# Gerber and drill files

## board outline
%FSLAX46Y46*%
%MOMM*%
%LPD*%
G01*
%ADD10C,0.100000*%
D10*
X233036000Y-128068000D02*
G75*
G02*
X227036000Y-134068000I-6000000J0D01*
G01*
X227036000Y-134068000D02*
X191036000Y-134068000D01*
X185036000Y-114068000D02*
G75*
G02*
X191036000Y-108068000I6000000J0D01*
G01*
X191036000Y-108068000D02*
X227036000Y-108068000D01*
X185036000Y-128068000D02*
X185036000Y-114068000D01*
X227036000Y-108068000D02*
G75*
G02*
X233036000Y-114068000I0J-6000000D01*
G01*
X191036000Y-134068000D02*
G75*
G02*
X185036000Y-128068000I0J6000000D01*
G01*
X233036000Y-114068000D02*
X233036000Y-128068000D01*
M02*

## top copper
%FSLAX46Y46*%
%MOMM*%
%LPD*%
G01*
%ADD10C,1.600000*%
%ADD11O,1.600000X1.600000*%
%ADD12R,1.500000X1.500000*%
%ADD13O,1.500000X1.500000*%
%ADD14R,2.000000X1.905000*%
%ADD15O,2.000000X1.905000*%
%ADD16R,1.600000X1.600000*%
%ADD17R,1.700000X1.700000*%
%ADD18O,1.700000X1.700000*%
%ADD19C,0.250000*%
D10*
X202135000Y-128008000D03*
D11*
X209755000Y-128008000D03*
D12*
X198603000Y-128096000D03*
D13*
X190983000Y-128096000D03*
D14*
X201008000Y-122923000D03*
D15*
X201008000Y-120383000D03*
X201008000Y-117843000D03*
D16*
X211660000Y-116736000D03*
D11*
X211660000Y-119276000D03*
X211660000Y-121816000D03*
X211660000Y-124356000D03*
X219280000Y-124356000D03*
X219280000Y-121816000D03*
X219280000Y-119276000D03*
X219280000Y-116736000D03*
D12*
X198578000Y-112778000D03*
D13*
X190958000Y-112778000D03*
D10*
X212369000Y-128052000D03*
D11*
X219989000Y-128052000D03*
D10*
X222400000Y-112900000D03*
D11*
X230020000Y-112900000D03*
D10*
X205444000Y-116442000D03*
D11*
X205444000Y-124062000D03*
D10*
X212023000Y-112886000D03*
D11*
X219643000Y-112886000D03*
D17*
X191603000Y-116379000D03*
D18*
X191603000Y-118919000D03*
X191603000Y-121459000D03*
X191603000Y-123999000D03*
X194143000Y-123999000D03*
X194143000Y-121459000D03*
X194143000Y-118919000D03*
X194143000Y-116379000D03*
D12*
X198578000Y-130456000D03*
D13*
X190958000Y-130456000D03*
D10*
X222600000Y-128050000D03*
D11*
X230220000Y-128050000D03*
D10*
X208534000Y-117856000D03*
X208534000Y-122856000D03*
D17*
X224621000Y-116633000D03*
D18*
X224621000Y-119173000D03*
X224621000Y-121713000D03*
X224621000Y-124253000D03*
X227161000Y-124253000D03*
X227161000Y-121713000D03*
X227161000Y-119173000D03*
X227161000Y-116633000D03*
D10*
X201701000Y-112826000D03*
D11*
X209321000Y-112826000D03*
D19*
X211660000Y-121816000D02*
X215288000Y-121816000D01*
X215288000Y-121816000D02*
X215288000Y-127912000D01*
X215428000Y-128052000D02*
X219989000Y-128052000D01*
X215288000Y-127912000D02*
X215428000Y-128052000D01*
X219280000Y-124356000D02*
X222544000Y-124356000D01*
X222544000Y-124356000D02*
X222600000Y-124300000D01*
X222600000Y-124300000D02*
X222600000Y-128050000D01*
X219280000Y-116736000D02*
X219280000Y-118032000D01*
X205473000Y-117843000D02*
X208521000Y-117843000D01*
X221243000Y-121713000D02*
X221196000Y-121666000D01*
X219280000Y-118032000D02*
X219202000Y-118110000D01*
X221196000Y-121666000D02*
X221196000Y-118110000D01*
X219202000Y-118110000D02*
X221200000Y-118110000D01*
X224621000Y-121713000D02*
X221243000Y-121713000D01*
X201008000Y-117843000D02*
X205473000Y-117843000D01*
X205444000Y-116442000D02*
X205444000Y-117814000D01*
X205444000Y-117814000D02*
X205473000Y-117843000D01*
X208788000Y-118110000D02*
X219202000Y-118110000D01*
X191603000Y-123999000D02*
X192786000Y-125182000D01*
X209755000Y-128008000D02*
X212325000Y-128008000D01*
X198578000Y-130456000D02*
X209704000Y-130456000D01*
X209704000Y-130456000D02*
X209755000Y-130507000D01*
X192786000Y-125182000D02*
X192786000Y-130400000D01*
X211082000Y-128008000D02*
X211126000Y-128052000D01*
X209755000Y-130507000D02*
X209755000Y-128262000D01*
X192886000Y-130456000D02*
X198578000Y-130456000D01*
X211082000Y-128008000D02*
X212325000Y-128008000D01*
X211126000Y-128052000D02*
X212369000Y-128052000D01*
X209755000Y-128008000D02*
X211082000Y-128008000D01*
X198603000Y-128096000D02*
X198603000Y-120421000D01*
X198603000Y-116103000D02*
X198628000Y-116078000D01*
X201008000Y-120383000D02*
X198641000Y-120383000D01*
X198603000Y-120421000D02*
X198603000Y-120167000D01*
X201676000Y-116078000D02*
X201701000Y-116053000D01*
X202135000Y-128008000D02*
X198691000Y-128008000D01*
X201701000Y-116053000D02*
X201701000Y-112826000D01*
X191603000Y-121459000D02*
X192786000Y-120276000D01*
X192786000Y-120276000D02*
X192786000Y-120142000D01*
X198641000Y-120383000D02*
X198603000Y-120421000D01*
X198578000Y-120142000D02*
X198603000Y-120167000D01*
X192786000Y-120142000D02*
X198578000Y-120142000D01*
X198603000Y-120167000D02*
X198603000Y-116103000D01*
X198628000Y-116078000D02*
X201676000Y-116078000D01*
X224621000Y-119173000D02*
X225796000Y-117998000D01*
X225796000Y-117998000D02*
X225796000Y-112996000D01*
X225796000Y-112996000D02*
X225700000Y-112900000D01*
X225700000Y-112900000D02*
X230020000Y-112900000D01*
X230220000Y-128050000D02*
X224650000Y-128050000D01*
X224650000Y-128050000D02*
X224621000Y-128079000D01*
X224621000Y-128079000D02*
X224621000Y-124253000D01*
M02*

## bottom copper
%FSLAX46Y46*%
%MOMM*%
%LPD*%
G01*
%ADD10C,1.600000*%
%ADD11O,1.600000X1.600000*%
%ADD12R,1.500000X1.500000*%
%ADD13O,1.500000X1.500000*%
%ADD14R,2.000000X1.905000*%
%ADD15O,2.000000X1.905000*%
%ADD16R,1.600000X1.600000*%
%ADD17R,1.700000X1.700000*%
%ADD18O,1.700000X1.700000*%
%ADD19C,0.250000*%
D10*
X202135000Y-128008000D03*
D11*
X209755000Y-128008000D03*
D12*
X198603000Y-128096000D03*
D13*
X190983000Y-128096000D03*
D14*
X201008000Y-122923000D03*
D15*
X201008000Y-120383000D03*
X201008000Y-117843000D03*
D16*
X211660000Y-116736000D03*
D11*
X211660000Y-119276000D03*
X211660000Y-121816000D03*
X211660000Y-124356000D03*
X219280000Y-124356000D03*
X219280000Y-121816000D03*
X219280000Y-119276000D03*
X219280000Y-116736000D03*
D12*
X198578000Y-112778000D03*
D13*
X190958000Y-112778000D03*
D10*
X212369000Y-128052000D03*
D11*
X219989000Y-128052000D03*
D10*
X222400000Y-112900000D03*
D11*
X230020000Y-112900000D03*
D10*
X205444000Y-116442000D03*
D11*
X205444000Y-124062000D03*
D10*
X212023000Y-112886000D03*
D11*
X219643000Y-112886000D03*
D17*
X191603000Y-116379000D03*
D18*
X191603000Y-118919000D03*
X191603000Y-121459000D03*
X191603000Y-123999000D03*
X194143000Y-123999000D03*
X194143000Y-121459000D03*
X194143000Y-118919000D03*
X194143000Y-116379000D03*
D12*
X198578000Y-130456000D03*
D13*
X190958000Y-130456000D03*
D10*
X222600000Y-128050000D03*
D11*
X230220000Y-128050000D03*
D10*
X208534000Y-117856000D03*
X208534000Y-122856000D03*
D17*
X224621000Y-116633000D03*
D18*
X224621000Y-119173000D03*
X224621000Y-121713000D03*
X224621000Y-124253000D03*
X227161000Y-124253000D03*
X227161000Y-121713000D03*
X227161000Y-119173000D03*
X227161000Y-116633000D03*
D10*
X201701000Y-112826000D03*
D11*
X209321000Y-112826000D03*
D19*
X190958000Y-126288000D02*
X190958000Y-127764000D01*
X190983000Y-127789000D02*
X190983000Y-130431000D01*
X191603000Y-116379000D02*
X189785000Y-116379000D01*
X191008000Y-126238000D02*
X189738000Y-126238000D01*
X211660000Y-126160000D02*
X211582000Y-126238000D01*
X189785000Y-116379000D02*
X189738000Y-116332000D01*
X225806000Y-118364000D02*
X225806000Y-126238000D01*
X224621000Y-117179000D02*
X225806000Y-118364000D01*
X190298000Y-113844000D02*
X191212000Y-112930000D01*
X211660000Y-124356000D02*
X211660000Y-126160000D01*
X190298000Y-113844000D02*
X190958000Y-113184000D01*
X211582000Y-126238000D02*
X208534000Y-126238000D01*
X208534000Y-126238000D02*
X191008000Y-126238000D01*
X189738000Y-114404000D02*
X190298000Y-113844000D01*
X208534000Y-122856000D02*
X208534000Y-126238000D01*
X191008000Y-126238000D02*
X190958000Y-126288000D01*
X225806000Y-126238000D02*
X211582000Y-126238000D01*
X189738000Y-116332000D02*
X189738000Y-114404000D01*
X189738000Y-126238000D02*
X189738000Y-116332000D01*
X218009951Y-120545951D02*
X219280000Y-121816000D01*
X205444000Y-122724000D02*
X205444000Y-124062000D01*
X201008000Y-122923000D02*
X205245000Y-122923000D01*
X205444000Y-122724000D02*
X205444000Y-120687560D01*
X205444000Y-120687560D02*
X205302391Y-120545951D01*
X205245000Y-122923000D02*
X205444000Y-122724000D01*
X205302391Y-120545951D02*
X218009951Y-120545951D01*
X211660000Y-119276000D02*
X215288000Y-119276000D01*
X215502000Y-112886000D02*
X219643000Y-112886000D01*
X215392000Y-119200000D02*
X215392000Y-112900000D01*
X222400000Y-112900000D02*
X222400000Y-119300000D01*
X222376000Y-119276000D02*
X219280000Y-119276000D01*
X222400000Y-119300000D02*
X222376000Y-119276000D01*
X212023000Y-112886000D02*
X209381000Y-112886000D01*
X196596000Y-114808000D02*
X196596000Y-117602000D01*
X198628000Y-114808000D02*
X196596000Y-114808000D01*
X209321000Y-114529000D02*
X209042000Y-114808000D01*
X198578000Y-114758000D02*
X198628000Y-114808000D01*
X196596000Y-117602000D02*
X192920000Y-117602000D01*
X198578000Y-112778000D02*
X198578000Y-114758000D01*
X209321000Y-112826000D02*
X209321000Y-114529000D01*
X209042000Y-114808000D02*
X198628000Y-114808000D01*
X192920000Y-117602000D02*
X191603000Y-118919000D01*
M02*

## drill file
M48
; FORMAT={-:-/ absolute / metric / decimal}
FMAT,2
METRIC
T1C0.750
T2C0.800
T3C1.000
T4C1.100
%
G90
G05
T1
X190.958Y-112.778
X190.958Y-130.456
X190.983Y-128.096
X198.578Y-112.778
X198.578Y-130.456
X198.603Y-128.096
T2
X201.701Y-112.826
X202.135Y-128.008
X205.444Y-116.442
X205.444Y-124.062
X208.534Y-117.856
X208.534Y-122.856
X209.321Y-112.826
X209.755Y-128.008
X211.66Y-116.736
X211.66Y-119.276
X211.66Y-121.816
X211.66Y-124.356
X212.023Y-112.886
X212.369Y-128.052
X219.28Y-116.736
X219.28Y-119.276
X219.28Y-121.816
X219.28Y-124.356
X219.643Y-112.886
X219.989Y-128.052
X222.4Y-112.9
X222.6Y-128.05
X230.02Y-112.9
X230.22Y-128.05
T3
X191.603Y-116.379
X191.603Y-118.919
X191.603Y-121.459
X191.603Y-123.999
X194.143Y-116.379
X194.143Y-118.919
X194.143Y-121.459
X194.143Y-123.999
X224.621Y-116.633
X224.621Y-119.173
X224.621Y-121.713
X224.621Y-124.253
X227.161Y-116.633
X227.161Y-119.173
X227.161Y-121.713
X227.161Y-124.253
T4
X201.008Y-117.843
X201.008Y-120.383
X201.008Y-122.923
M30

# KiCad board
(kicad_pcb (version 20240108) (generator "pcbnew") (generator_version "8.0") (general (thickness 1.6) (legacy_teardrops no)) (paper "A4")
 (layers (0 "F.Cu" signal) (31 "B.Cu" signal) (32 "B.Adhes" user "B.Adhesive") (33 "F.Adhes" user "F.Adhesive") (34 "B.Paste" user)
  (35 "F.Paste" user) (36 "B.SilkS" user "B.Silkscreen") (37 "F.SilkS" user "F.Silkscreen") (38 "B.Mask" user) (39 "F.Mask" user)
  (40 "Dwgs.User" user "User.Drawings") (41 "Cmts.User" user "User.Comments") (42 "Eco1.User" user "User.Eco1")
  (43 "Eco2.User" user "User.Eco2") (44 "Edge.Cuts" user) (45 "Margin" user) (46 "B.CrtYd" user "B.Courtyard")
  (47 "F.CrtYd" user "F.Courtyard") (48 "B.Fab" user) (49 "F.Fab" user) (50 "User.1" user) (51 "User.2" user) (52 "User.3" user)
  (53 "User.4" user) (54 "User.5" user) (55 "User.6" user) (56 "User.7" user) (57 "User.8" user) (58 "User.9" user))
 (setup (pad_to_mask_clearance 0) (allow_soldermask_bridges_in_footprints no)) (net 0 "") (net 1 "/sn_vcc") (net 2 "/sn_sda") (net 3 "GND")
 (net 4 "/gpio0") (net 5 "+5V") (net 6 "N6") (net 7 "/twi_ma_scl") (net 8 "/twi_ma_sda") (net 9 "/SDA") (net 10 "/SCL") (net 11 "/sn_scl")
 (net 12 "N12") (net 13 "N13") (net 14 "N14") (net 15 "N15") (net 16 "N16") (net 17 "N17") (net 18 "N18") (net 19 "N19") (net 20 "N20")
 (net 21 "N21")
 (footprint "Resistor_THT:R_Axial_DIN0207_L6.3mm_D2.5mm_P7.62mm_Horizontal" (layer "F.Cu") (at 202.135 128.008)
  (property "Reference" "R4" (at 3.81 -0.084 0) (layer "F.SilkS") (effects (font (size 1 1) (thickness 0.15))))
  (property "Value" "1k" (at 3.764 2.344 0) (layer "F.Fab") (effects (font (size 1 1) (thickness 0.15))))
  (pad "1" thru_hole circle (at 0 0) (size 1.6 1.6) (drill 0.8) (layers "*.Cu" "*.Mask") (remove_unused_layers no) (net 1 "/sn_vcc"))
  (pad "2" thru_hole oval (at 7.62 0) (size 1.6 1.6) (drill 0.8) (layers "*.Cu" "*.Mask") (remove_unused_layers no) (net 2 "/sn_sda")))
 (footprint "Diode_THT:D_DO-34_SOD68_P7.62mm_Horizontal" (layer "F.Cu") (at 198.603 128.096 180)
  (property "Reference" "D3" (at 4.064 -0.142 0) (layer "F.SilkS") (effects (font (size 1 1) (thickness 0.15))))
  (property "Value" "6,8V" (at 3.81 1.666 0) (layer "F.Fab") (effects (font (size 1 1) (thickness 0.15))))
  (pad "1" thru_hole rect (at 0 0 180) (size 1.5 1.5) (drill 0.75) (layers "*.Cu" "*.Mask") (remove_unused_layers no) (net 1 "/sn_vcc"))
  (pad "2" thru_hole oval (at 7.62 0 180) (size 1.5 1.5) (drill 0.75) (layers "*.Cu" "*.Mask") (remove_unused_layers no) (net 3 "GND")))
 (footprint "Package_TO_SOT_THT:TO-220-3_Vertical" (layer "F.Cu") (at 201.008 122.923 90)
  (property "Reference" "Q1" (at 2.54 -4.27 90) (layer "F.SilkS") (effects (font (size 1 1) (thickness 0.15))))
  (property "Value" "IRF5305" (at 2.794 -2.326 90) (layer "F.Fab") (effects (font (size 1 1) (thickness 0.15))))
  (pad "1" thru_hole rect (at 0 0 90) (size 1.905 2) (drill 1.1) (layers "*.Cu" "*.Mask") (remove_unused_layers no) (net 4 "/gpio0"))
  (pad "2" thru_hole oval (at 2.54 0 90) (size 1.905 2) (drill 1.1) (layers "*.Cu" "*.Mask") (remove_unused_layers no) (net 1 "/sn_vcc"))
  (pad "3" thru_hole oval (at 5.08 0 90) (size 1.905 2) (drill 1.1) (layers "*.Cu" "*.Mask") (remove_unused_layers no) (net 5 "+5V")))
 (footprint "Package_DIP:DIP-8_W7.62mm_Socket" (layer "F.Cu") (at 211.66 116.736)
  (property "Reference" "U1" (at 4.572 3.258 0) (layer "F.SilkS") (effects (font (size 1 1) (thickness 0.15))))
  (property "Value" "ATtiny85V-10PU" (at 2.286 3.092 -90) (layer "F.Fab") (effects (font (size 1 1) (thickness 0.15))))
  (pad "1" thru_hole rect (at 0 0) (size 1.6 1.6) (drill 0.8) (layers "*.Cu" "*.Mask") (remove_unused_layers no) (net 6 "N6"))
  (pad "2" thru_hole oval (at 0 2.54) (size 1.6 1.6) (drill 0.8) (layers "*.Cu" "*.Mask") (remove_unused_layers no) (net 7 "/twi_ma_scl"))
  (pad "3" thru_hole oval (at 0 5.08) (size 1.6 1.6) (drill 0.8) (layers "*.Cu" "*.Mask") (remove_unused_layers no) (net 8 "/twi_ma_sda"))
  (pad "4" thru_hole oval (at 0 7.62) (size 1.6 1.6) (drill 0.8) (layers "*.Cu" "*.Mask") (remove_unused_layers no) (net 3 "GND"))
  (pad "5" thru_hole oval (at 7.62 7.62) (size 1.6 1.6) (drill 0.8) (layers "*.Cu" "*.Mask") (remove_unused_layers no) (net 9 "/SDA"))
  (pad "6" thru_hole oval (at 7.62 5.08) (size 1.6 1.6) (drill 0.8) (layers "*.Cu" "*.Mask") (remove_unused_layers no) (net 4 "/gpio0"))
  (pad "7" thru_hole oval (at 7.62 2.54) (size 1.6 1.6) (drill 0.8) (layers "*.Cu" "*.Mask") (remove_unused_layers no) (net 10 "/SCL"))
  (pad "8" thru_hole oval (at 7.62 0) (size 1.6 1.6) (drill 0.8) (layers "*.Cu" "*.Mask") (remove_unused_layers no) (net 5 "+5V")))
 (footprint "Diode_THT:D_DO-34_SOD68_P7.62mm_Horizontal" (layer "F.Cu") (at 198.578 112.778 180)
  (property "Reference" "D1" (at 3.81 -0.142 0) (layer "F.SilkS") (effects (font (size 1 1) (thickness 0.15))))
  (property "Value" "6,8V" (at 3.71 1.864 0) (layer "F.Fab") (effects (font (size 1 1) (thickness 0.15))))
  (pad "1" thru_hole rect (at 0 0 180) (size 1.5 1.5) (drill 0.75) (layers "*.Cu" "*.Mask") (remove_unused_layers no) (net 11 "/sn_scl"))
  (pad "2" thru_hole oval (at 7.62 0 180) (size 1.5 1.5) (drill 0.75) (layers "*.Cu" "*.Mask") (remove_unused_layers no) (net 3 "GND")))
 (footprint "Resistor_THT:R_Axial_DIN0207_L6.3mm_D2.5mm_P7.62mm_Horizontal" (layer "F.Cu") (at 212.369 128.052)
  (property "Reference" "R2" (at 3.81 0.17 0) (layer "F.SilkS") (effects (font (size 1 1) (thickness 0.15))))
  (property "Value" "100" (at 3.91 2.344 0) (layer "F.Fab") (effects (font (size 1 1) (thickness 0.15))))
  (pad "1" thru_hole circle (at 0 0) (size 1.6 1.6) (drill 0.8) (layers "*.Cu" "*.Mask") (remove_unused_layers no) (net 2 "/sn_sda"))
  (pad "2" thru_hole oval (at 7.62 0) (size 1.6 1.6) (drill 0.8) (layers "*.Cu" "*.Mask") (remove_unused_layers no) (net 8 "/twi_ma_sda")))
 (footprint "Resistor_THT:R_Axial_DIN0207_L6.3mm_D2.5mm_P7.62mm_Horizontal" (layer "F.Cu") (at 222.4 112.9)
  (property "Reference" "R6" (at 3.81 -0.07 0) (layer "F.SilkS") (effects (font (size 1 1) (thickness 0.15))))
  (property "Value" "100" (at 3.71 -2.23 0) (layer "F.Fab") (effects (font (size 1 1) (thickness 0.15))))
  (pad "1" thru_hole circle (at 0 0) (size 1.6 1.6) (drill 0.8) (layers "*.Cu" "*.Mask") (remove_unused_layers no) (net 10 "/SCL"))
  (pad "2" thru_hole oval (at 7.62 0) (size 1.6 1.6) (drill 0.8) (layers "*.Cu" "*.Mask") (remove_unused_layers no) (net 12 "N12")))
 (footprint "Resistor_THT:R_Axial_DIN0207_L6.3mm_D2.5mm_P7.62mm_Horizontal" (layer "F.Cu") (at 205.444 116.442 -90)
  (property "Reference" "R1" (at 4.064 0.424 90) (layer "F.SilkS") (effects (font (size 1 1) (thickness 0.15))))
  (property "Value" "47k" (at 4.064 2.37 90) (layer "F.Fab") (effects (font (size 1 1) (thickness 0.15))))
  (pad "1" thru_hole circle (at 0 0 270) (size 1.6 1.6) (drill 0.8) (layers "*.Cu" "*.Mask") (remove_unused_layers no) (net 5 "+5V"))
  (pad "2" thru_hole oval (at 7.62 0 270) (size 1.6 1.6) (drill 0.8) (layers "*.Cu" "*.Mask") (remove_unused_layers no) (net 4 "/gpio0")))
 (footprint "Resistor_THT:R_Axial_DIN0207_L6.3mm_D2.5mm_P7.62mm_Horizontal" (layer "F.Cu") (at 212.023 112.886)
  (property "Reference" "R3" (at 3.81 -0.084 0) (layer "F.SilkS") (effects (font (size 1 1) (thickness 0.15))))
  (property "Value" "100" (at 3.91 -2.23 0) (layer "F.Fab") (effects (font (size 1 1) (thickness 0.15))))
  (pad "1" thru_hole circle (at 0 0) (size 1.6 1.6) (drill 0.8) (layers "*.Cu" "*.Mask") (remove_unused_layers no) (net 11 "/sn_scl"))
  (pad "2" thru_hole oval (at 7.62 0) (size 1.6 1.6) (drill 0.8) (layers "*.Cu" "*.Mask") (remove_unused_layers no) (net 7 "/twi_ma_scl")))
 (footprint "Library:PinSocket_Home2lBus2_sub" (layer "F.Cu") (at 194.103 116.379)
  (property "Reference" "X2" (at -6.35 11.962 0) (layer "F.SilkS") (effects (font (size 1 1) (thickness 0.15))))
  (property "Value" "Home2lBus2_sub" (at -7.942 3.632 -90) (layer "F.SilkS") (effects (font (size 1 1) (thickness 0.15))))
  (pad "1" thru_hole rect (at -2.5 0) (size 1.7 1.7) (drill 1) (layers "*.Cu" "*.Mask") (remove_unused_layers no) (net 3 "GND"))
  (pad "2" thru_hole oval (at -2.5 2.54) (size 1.7 1.7) (drill 1) (layers "*.Cu" "*.Mask") (remove_unused_layers no) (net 11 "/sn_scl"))
  (pad "3" thru_hole oval (at -2.5 5.08) (size 1.7 1.7) (drill 1) (layers "*.Cu" "*.Mask") (remove_unused_layers no) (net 1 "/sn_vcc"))
  (pad "4" thru_hole oval (at -2.5 7.62) (size 1.7 1.7) (drill 1) (layers "*.Cu" "*.Mask") (remove_unused_layers no) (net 2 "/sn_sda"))
  (pad "5" thru_hole oval (at 0.04 7.62) (size 1.7 1.7) (drill 1) (layers "*.Cu" "*.Mask") (remove_unused_layers no) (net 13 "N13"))
  (pad "6" thru_hole oval (at 0.04 5.08) (size 1.7 1.7) (drill 1) (layers "*.Cu" "*.Mask") (remove_unused_layers no) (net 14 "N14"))
  (pad "7" thru_hole oval (at 0.04 2.54) (size 1.7 1.7) (drill 1) (layers "*.Cu" "*.Mask") (remove_unused_layers no) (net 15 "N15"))
  (pad "8" thru_hole oval (at 0.04 0) (size 1.7 1.7) (drill 1) (layers "*.Cu" "*.Mask") (remove_unused_layers no) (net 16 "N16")))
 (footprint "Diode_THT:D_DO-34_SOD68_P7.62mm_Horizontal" (layer "F.Cu") (at 198.578 130.456 180)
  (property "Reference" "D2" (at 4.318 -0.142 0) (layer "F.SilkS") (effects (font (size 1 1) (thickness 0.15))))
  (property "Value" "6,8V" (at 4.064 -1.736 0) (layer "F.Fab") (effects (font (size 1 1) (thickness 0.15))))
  (pad "1" thru_hole rect (at 0 0 180) (size 1.5 1.5) (drill 0.75) (layers "*.Cu" "*.Mask") (remove_unused_layers no) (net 2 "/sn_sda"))
  (pad "2" thru_hole oval (at 7.62 0 180) (size 1.5 1.5) (drill 0.75) (layers "*.Cu" "*.Mask") (remove_unused_layers no) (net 3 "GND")))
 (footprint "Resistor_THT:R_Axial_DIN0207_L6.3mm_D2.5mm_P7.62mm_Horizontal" (layer "F.Cu") (at 222.6 128.05)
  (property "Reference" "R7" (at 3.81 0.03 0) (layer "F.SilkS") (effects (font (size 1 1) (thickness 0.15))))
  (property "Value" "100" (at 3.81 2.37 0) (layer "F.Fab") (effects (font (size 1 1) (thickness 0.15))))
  (pad "1" thru_hole circle (at 0 0) (size 1.6 1.6) (drill 0.8) (layers "*.Cu" "*.Mask") (remove_unused_layers no) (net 9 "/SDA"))
  (pad "2" thru_hole oval (at 7.62 0) (size 1.6 1.6) (drill 0.8) (layers "*.Cu" "*.Mask") (remove_unused_layers no) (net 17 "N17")))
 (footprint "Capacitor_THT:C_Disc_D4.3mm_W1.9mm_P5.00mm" (layer "F.Cu") (at 208.534 117.856 -90)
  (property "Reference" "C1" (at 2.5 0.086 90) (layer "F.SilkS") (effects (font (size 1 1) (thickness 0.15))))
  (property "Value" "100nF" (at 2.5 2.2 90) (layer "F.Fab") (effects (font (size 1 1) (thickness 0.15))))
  (pad "1" thru_hole circle (at 0 0 270) (size 1.6 1.6) (drill 0.8) (layers "*.Cu" "*.Mask") (remove_unused_layers no) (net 5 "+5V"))
  (pad "2" thru_hole circle (at 5 0 270) (size 1.6 1.6) (drill 0.8) (layers "*.Cu" "*.Mask") (remove_unused_layers no) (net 3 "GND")))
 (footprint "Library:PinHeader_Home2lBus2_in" (layer "F.Cu") (at 224.621 116.633)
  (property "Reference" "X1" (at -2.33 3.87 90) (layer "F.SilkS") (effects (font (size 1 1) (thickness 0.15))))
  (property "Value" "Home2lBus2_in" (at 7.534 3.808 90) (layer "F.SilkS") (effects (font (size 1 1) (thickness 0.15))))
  (pad "1" thru_hole rect (at 0 0) (size 1.7 1.7) (drill 1) (layers "*.Cu" "*.Mask") (remove_unused_layers no) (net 3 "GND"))
  (pad "2" thru_hole oval (at 0 2.54) (size 1.7 1.7) (drill 1) (layers "*.Cu" "*.Mask") (remove_unused_layers no) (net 12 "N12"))
  (pad "3" thru_hole oval (at 0 5.08) (size 1.7 1.7) (drill 1) (layers "*.Cu" "*.Mask") (remove_unused_layers no) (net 5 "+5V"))
  (pad "4" thru_hole oval (at 0 7.62) (size 1.7 1.7) (drill 1) (layers "*.Cu" "*.Mask") (remove_unused_layers no) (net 17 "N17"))
  (pad "5" thru_hole oval (at 2.54 7.62) (size 1.7 1.7) (drill 1) (layers "*.Cu" "*.Mask") (remove_unused_layers no) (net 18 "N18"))
  (pad "6" thru_hole oval (at 2.54 5.08) (size 1.7 1.7) (drill 1) (layers "*.Cu" "*.Mask") (remove_unused_layers no) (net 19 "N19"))
  (pad "7" thru_hole oval (at 2.54 2.54) (size 1.7 1.7) (drill 1) (layers "*.Cu" "*.Mask") (remove_unused_layers no) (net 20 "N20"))
  (pad "8" thru_hole oval (at 2.54 0) (size 1.7 1.7) (drill 1) (layers "*.Cu" "*.Mask") (remove_unused_layers no) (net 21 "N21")))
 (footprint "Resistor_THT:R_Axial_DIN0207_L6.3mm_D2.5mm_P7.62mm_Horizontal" (layer "F.Cu") (at 201.701 112.826)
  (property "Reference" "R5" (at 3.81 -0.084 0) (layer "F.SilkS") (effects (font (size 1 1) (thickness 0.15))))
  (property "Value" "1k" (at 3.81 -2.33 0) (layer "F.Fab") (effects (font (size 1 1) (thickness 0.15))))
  (pad "1" thru_hole circle (at 0 0) (size 1.6 1.6) (drill 0.8) (layers "*.Cu" "*.Mask") (remove_unused_layers no) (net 1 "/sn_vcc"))
  (pad "2" thru_hole oval (at 7.62 0) (size 1.6 1.6) (drill 0.8) (layers "*.Cu" "*.Mask") (remove_unused_layers no) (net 11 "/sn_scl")))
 (gr_arc (start 233.036 128.068) (mid 231.278641 132.310641) (end 227.036 134.068) (stroke (width 0.1) (type solid)) (layer "Edge.Cuts"))
 (gr_line (start 227.036 134.068) (end 191.036 134.068) (stroke (width 0.1) (type solid)) (layer "Edge.Cuts"))
 (gr_arc (start 185.036 114.068) (mid 186.793359 109.825359) (end 191.036 108.068) (stroke (width 0.1) (type solid)) (layer "Edge.Cuts"))
 (gr_line (start 191.036 108.068) (end 227.036 108.068) (stroke (width 0.1) (type solid)) (layer "Edge.Cuts"))
 (gr_line (start 185.036 128.068) (end 185.036 114.068) (stroke (width 0.1) (type solid)) (layer "Edge.Cuts"))
 (gr_arc (start 227.036 108.068) (mid 231.278641 109.825359) (end 233.036 114.068) (stroke (width 0.1) (type solid)) (layer "Edge.Cuts"))
 (gr_arc (start 191.036 134.068) (mid 186.793359 132.310641) (end 185.036 128.068) (stroke (width 0.1) (type solid)) (layer "Edge.Cuts"))
 (gr_line (start 233.036 114.068) (end 233.036 128.068) (stroke (width 0.1) (type solid)) (layer "Edge.Cuts"))
 (segment (start 190.958 126.288) (end 190.958 127.764) (width 0.25) (layer "B.Cu") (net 3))
 (segment (start 190.983 127.789) (end 190.983 130.431) (width 0.25) (layer "B.Cu") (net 3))
 (segment (start 191.603 116.379) (end 189.785 116.379) (width 0.25) (layer "B.Cu") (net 3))
 (segment (start 191.008 126.238) (end 189.738 126.238) (width 0.25) (layer "B.Cu") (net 3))
 (segment (start 211.66 126.16) (end 211.582 126.238) (width 0.25) (layer "B.Cu") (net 3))
 (segment (start 189.785 116.379) (end 189.738 116.332) (width 0.25) (layer "B.Cu") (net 3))
 (segment (start 225.806 118.364) (end 225.806 126.238) (width 0.25) (layer "B.Cu") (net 3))
 (segment (start 224.621 117.179) (end 225.806 118.364) (width 0.25) (layer "B.Cu") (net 3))
 (segment (start 190.298 113.844) (end 191.212 112.93) (width 0.25) (layer "B.Cu") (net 3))
 (segment (start 211.66 124.356) (end 211.66 126.16) (width 0.25) (layer "B.Cu") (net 3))
 (segment (start 190.298 113.844) (end 190.958 113.184) (width 0.25) (layer "B.Cu") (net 3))
 (segment (start 211.582 126.238) (end 208.534 126.238) (width 0.25) (layer "B.Cu") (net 3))
 (segment (start 208.534 126.238) (end 191.008 126.238) (width 0.25) (layer "B.Cu") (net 3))
 (segment (start 189.738 114.404) (end 190.298 113.844) (width 0.25) (layer "B.Cu") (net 3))
 (segment (start 208.534 122.856) (end 208.534 126.238) (width 0.25) (layer "B.Cu") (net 3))
 (segment (start 191.008 126.238) (end 190.958 126.288) (width 0.25) (layer "B.Cu") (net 3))
 (segment (start 225.806 126.238) (end 211.582 126.238) (width 0.25) (layer "B.Cu") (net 3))
 (segment (start 189.738 116.332) (end 189.738 114.404) (width 0.25) (layer "B.Cu") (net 3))
 (segment (start 189.738 126.238) (end 189.738 116.332) (width 0.25) (layer "B.Cu") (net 3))
 (segment (start 218.009951 120.545951) (end 219.28 121.816) (width 0.25) (layer "B.Cu") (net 4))
 (segment (start 205.444 122.724) (end 205.444 124.062) (width 0.25) (layer "B.Cu") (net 4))
 (segment (start 201.008 122.923) (end 205.245 122.923) (width 0.25) (layer "B.Cu") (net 4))
 (segment (start 205.444 122.724) (end 205.444 120.68756) (width 0.25) (layer "B.Cu") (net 4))
 (segment (start 205.444 120.68756) (end 205.302391 120.545951) (width 0.25) (layer "B.Cu") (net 4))
 (segment (start 205.245 122.923) (end 205.444 122.724) (width 0.25) (layer "B.Cu") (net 4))
 (segment (start 205.302391 120.545951) (end 218.009951 120.545951) (width 0.25) (layer "B.Cu") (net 4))
 (segment (start 211.66 121.816) (end 215.288 121.816) (width 0.25) (layer "F.Cu") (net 8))
 (segment (start 215.288 121.816) (end 215.288 127.912) (width 0.25) (layer "F.Cu") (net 8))
 (segment (start 215.428 128.052) (end 219.989 128.052) (width 0.25) (layer "F.Cu") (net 8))
 (segment (start 215.288 127.912) (end 215.428 128.052) (width 0.25) (layer "F.Cu") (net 8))
 (segment (start 211.66 119.276) (end 215.288 119.276) (width 0.25) (layer "B.Cu") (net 7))
 (segment (start 215.502 112.886) (end 219.643 112.886) (width 0.25) (layer "B.Cu") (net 7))
 (segment (start 215.392 119.2) (end 215.392 112.9) (width 0.25) (layer "B.Cu") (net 7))
 (segment (start 219.28 124.356) (end 222.544 124.356) (width 0.25) (layer "F.Cu") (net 9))
 (segment (start 222.544 124.356) (end 222.6 124.3) (width 0.25) (layer "F.Cu") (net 9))
 (segment (start 222.6 124.3) (end 222.6 128.05) (width 0.25) (layer "F.Cu") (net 9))
 (segment (start 222.4 112.9) (end 222.4 119.3) (width 0.25) (layer "B.Cu") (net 10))
 (segment (start 222.376 119.276) (end 219.28 119.276) (width 0.25) (layer "B.Cu") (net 10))
 (segment (start 222.4 119.3) (end 222.376 119.276) (width 0.25) (layer "B.Cu") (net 10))
 (segment (start 219.28 116.736) (end 219.28 118.032) (width 0.25) (layer "F.Cu") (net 5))
 (segment (start 205.473 117.843) (end 208.521 117.843) (width 0.25) (layer "F.Cu") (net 5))
 (segment (start 221.243 121.713) (end 221.196 121.666) (width 0.25) (layer "F.Cu") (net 5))
 (segment (start 219.28 118.032) (end 219.202 118.11) (width 0.25) (layer "F.Cu") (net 5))
 (segment (start 221.196 121.666) (end 221.196 118.11) (width 0.25) (layer "F.Cu") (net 5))
 (segment (start 219.202 118.11) (end 221.2 118.11) (width 0.25) (layer "F.Cu") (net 5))
 (segment (start 224.621 121.713) (end 221.243 121.713) (width 0.25) (layer "F.Cu") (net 5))
 (segment (start 201.008 117.843) (end 205.473 117.843) (width 0.25) (layer "F.Cu") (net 5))
 (segment (start 205.444 116.442) (end 205.444 117.814) (width 0.25) (layer "F.Cu") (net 5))
 (segment (start 205.444 117.814) (end 205.473 117.843) (width 0.25) (layer "F.Cu") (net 5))
 (segment (start 208.788 118.11) (end 219.202 118.11) (width 0.25) (layer "F.Cu") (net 5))
 (segment (start 212.023 112.886) (end 209.381 112.886) (width 0.25) (layer "B.Cu") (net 11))
 (segment (start 196.596 114.808) (end 196.596 117.602) (width 0.25) (layer "B.Cu") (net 11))
 (segment (start 198.628 114.808) (end 196.596 114.808) (width 0.25) (layer "B.Cu") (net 11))
 (segment (start 209.321 114.529) (end 209.042 114.808) (width 0.25) (layer "B.Cu") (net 11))
 (segment (start 198.578 114.758) (end 198.628 114.808) (width 0.25) (layer "B.Cu") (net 11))
 (segment (start 196.596 117.602) (end 192.92 117.602) (width 0.25) (layer "B.Cu") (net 11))
 (segment (start 198.578 112.778) (end 198.578 114.758) (width 0.25) (layer "B.Cu") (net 11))
 (segment (start 209.321 112.826) (end 209.321 114.529) (width 0.25) (layer "B.Cu") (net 11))
 (segment (start 209.042 114.808) (end 198.628 114.808) (width 0.25) (layer "B.Cu") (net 11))
 (segment (start 192.92 117.602) (end 191.603 118.919) (width 0.25) (layer "B.Cu") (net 11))
 (segment (start 191.603 123.999) (end 192.786 125.182) (width 0.25) (layer "F.Cu") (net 2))
 (segment (start 209.755 128.008) (end 212.325 128.008) (width 0.25) (layer "F.Cu") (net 2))
 (segment (start 198.578 130.456) (end 209.704 130.456) (width 0.25) (layer "F.Cu") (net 2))
 (segment (start 209.704 130.456) (end 209.755 130.507) (width 0.25) (layer "F.Cu") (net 2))
 (segment (start 192.786 125.182) (end 192.786 130.4) (width 0.25) (layer "F.Cu") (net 2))
 (segment (start 211.082 128.008) (end 211.126 128.052) (width 0.25) (layer "F.Cu") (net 2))
 (segment (start 209.755 130.507) (end 209.755 128.262) (width 0.25) (layer "F.Cu") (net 2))
 (segment (start 192.886 130.456) (end 198.578 130.456) (width 0.25) (layer "F.Cu") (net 2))
 (segment (start 211.082 128.008) (end 212.325 128.008) (width 0.25) (layer "F.Cu") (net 2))
 (segment (start 211.126 128.052) (end 212.369 128.052) (width 0.25) (layer "F.Cu") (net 2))
 (segment (start 209.755 128.008) (end 211.082 128.008) (width 0.25) (layer "F.Cu") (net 2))
 (segment (start 198.603 128.096) (end 198.603 120.421) (width 0.25) (layer "F.Cu") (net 1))
 (segment (start 198.603 116.103) (end 198.628 116.078) (width 0.25) (layer "F.Cu") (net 1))
 (segment (start 201.008 120.383) (end 198.641 120.383) (width 0.25) (layer "F.Cu") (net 1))
 (segment (start 198.603 120.421) (end 198.603 120.167) (width 0.25) (layer "F.Cu") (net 1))
 (segment (start 201.676 116.078) (end 201.701 116.053) (width 0.25) (layer "F.Cu") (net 1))
 (segment (start 202.135 128.008) (end 198.691 128.008) (width 0.25) (layer "F.Cu") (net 1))
 (segment (start 201.701 116.053) (end 201.701 112.826) (width 0.25) (layer "F.Cu") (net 1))
 (segment (start 191.603 121.459) (end 192.786 120.276) (width 0.25) (layer "F.Cu") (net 1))
 (segment (start 192.786 120.276) (end 192.786 120.142) (width 0.25) (layer "F.Cu") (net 1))
 (segment (start 198.641 120.383) (end 198.603 120.421) (width 0.25) (layer "F.Cu") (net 1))
 (segment (start 198.578 120.142) (end 198.603 120.167) (width 0.25) (layer "F.Cu") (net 1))
 (segment (start 192.786 120.142) (end 198.578 120.142) (width 0.25) (layer "F.Cu") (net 1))
 (segment (start 198.603 120.167) (end 198.603 116.103) (width 0.25) (layer "F.Cu") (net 1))
 (segment (start 198.628 116.078) (end 201.676 116.078) (width 0.25) (layer "F.Cu") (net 1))
 (segment (start 224.621 119.173) (end 225.796 117.998) (width 0.25) (layer "F.Cu") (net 12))
 (segment (start 225.796 117.998) (end 225.796 112.996) (width 0.25) (layer "F.Cu") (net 12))
 (segment (start 225.796 112.996) (end 225.7 112.9) (width 0.25) (layer "F.Cu") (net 12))
 (segment (start 225.7 112.9) (end 230.02 112.9) (width 0.25) (layer "F.Cu") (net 12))
 (segment (start 230.22 128.05) (end 224.65 128.05) (width 0.25) (layer "F.Cu") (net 17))
 (segment (start 224.65 128.05) (end 224.621 128.079) (width 0.25) (layer "F.Cu") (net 17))
 (segment (start 224.621 128.079) (end 224.621 124.253) (width 0.25) (layer "F.Cu") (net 17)))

